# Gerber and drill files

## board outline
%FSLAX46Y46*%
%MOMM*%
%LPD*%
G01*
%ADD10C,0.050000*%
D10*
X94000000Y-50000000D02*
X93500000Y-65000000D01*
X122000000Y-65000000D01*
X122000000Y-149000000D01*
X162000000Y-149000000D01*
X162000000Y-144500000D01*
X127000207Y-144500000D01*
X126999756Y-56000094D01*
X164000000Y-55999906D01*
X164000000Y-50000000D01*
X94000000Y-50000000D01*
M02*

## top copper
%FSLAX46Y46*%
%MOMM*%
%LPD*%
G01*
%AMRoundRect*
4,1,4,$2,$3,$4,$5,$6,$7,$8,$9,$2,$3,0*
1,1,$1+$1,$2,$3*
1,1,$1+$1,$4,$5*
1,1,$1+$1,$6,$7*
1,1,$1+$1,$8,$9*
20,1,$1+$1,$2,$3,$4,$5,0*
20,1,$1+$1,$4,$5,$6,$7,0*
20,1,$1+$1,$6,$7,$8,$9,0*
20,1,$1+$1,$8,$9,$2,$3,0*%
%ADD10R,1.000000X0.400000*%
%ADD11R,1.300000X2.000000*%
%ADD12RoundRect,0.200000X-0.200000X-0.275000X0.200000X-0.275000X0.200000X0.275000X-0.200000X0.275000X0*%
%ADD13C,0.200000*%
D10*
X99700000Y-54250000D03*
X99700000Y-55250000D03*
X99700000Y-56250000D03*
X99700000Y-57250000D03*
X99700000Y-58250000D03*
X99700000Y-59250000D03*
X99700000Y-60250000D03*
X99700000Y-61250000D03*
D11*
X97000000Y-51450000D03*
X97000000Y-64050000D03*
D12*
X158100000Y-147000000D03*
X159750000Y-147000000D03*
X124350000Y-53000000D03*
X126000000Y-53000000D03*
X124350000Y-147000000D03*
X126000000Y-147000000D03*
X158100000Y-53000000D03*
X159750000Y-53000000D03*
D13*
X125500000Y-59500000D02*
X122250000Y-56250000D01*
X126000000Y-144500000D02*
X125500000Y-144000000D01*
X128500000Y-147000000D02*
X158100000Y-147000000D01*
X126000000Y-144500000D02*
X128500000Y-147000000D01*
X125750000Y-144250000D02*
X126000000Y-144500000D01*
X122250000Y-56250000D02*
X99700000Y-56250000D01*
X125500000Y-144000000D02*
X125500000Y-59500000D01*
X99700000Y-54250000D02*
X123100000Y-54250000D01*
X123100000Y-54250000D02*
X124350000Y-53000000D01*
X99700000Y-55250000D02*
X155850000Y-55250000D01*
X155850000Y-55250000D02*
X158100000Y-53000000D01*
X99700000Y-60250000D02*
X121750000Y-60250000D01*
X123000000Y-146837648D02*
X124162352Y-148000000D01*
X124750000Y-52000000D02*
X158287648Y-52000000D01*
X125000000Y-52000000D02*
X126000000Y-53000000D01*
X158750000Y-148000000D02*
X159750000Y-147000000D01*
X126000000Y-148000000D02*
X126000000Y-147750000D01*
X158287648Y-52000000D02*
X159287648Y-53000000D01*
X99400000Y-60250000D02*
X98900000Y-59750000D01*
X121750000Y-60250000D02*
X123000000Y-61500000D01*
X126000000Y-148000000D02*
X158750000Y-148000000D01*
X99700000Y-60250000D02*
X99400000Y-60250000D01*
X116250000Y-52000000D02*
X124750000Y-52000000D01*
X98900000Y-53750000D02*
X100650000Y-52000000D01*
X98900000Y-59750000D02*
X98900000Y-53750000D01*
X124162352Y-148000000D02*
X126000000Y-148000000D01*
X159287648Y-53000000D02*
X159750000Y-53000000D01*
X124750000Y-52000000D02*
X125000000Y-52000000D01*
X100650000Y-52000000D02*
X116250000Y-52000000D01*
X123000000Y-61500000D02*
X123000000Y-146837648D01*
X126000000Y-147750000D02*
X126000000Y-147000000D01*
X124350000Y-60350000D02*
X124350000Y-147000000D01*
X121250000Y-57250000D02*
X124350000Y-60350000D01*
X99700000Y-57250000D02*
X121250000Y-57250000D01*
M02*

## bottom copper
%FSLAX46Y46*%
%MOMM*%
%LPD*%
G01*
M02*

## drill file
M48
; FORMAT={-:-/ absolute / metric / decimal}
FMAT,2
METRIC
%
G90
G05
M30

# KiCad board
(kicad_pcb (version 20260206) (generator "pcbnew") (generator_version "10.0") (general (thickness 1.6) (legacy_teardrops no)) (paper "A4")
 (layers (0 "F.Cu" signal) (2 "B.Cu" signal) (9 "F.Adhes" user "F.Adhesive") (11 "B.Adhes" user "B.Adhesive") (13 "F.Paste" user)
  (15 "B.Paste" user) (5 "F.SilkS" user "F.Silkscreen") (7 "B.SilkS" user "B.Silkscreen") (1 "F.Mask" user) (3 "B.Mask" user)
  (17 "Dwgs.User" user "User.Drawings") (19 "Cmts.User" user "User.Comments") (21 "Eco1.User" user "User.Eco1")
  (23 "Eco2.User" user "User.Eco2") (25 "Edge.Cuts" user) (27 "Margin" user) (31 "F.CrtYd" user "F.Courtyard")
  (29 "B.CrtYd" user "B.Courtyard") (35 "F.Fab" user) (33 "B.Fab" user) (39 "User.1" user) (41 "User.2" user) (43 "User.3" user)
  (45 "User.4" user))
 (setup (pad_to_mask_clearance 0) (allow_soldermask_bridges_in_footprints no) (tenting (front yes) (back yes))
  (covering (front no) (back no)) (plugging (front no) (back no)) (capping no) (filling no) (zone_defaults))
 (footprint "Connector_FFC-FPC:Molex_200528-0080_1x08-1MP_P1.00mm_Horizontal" (layer "F.Cu") (at 98.79 57.75 -90)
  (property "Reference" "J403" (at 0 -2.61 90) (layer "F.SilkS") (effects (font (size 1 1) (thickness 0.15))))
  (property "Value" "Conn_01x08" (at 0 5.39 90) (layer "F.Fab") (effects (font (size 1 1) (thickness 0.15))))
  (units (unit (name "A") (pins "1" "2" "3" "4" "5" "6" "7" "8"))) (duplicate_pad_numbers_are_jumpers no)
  (pad "1" smd rect (at -3.5 -0.91 270) (size 0.4 1) (layers "F.Cu" "F.Mask" "F.Paste") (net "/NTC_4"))
  (pad "2" smd rect (at -2.5 -0.91 270) (size 0.4 1) (layers "F.Cu" "F.Mask" "F.Paste") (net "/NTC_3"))
  (pad "3" smd rect (at -1.5 -0.91 270) (size 0.4 1) (layers "F.Cu" "F.Mask" "F.Paste") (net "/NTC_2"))
  (pad "4" smd rect (at -0.5 -0.91 270) (size 0.4 1) (layers "F.Cu" "F.Mask" "F.Paste") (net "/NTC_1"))
  (pad "5" smd rect (at 0.5 -0.91 270) (size 0.4 1) (layers "F.Cu" "F.Mask" "F.Paste") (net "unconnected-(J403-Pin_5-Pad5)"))
  (pad "6" smd rect (at 1.5 -0.91 270) (size 0.4 1) (layers "F.Cu" "F.Mask" "F.Paste") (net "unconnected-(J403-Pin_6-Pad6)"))
  (pad "7" smd rect (at 2.5 -0.91 270) (size 0.4 1) (layers "F.Cu" "F.Mask" "F.Paste") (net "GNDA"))
  (pad "8" smd rect (at 3.5 -0.91 270) (size 0.4 1) (layers "F.Cu" "F.Mask" "F.Paste") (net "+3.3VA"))
  (pad "MP" smd rect (at -6.3 1.79 270) (size 2 1.3) (layers "F.Cu" "F.Mask" "F.Paste"))
  (pad "MP" smd rect (at 6.3 1.79 270) (size 2 1.3) (layers "F.Cu" "F.Mask" "F.Paste")))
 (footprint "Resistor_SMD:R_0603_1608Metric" (layer "F.Cu") (at 158.925 147)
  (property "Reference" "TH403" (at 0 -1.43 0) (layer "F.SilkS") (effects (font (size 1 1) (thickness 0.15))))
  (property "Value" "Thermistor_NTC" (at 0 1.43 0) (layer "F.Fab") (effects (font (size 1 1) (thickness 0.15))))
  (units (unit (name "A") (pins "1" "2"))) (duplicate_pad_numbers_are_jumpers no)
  (pad "1" smd roundrect (at -0.825 0) (size 0.8 0.95) (layers "F.Cu" "F.Mask" "F.Paste") (roundrect_rratio 0.25) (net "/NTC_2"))
  (pad "2" smd roundrect (at 0.825 0) (size 0.8 0.95) (layers "F.Cu" "F.Mask" "F.Paste") (roundrect_rratio 0.25) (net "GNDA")))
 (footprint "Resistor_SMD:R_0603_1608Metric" (layer "F.Cu") (at 125.175 53)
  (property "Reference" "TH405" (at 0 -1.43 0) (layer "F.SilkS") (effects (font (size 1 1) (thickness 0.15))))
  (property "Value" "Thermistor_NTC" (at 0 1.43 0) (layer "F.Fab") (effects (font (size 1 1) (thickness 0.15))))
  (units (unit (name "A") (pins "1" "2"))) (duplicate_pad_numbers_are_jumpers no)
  (pad "1" smd roundrect (at -0.825 0) (size 0.8 0.95) (layers "F.Cu" "F.Mask" "F.Paste") (roundrect_rratio 0.25) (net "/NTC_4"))
  (pad "2" smd roundrect (at 0.825 0) (size 0.8 0.95) (layers "F.Cu" "F.Mask" "F.Paste") (roundrect_rratio 0.25) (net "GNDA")))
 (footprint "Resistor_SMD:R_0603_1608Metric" (layer "F.Cu") (at 125.175 147)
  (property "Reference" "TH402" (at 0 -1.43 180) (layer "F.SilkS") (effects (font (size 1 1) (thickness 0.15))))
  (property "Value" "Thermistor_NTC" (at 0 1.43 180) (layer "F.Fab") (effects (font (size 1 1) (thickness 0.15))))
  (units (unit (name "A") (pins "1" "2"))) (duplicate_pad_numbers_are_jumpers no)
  (pad "1" smd roundrect (at -0.825 0) (size 0.8 0.95) (layers "F.Cu" "F.Mask" "F.Paste") (roundrect_rratio 0.25) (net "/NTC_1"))
  (pad "2" smd roundrect (at 0.825 0) (size 0.8 0.95) (layers "F.Cu" "F.Mask" "F.Paste") (roundrect_rratio 0.25) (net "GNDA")))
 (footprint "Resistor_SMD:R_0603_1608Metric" (layer "F.Cu") (at 158.925 53)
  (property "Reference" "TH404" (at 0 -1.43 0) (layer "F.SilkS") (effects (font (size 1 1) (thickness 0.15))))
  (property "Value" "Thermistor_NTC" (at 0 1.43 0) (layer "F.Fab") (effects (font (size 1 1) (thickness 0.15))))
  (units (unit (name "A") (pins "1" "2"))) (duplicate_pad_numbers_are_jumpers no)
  (pad "1" smd roundrect (at -0.825 0) (size 0.8 0.95) (layers "F.Cu" "F.Mask" "F.Paste") (roundrect_rratio 0.25) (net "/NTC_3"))
  (pad "2" smd roundrect (at 0.825 0) (size 0.8 0.95) (layers "F.Cu" "F.Mask" "F.Paste") (roundrect_rratio 0.25) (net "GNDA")))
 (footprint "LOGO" (layer "F.Cu") (at 109 57)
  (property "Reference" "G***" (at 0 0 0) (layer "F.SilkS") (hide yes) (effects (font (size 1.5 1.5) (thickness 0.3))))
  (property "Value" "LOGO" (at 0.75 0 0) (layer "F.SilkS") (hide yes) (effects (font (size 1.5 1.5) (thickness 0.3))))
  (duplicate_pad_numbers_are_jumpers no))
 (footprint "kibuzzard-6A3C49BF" (layer "B.Cu") (at 96.5 57.5 90)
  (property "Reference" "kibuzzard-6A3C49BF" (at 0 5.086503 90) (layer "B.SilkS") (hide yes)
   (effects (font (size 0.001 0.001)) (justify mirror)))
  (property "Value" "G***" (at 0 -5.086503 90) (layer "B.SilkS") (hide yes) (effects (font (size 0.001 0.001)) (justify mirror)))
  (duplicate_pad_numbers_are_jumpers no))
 (gr_poly
  (pts (xy 94 50) (xy 93.5 65) (xy 122 65) (xy 122 149) (xy 162 149) (xy 162 144.5) (xy 127.000207 144.5) (xy 126.999756 56.000094)
   (xy 164 55.999906) (xy 164 50))
  (stroke (width 0.05) (type solid)) (fill no) (layer "Edge.Cuts"))
 (segment (start 125.5 59.5) (end 122.25 56.25) (width 0.2) (layer "F.Cu") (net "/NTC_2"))
 (segment (start 126 144.5) (end 125.5 144) (width 0.2) (layer "F.Cu") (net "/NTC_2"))
 (segment (start 128.5 147) (end 158.1 147) (width 0.2) (layer "F.Cu") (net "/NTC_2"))
 (segment (start 126 144.5) (end 128.5 147) (width 0.2) (layer "F.Cu") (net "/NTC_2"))
 (segment (start 125.75 144.25) (end 126 144.5) (width 0.2) (layer "F.Cu") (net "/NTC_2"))
 (segment (start 122.25 56.25) (end 99.7 56.25) (width 0.2) (layer "F.Cu") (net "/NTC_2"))
 (segment (start 125.5 144) (end 125.5 59.5) (width 0.2) (layer "F.Cu") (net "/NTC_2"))
 (segment (start 99.7 54.25) (end 123.1 54.25) (width 0.2) (layer "F.Cu") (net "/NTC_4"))
 (segment (start 123.1 54.25) (end 124.35 53) (width 0.2) (layer "F.Cu") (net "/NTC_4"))
 (segment (start 99.7 55.25) (end 155.85 55.25) (width 0.2) (layer "F.Cu") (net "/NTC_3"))
 (segment (start 155.85 55.25) (end 158.1 53) (width 0.2) (layer "F.Cu") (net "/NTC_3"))
 (segment (start 99.7 60.25) (end 121.75 60.25) (width 0.2) (layer "F.Cu") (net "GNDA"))
 (segment (start 123 146.837648) (end 124.162352 148) (width 0.2) (layer "F.Cu") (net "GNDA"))
 (segment (start 124.75 52) (end 158.287648 52) (width 0.2) (layer "F.Cu") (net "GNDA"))
 (segment (start 125 52) (end 126 53) (width 0.2) (layer "F.Cu") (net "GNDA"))
 (segment (start 158.75 148) (end 159.75 147) (width 0.2) (layer "F.Cu") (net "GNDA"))
 (segment (start 126 148) (end 126 147.75) (width 0.2) (layer "F.Cu") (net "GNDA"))
 (segment (start 158.287648 52) (end 159.287648 53) (width 0.2) (layer "F.Cu") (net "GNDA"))
 (segment (start 99.4 60.25) (end 98.9 59.75) (width 0.2) (layer "F.Cu") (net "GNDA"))
 (segment (start 121.75 60.25) (end 123 61.5) (width 0.2) (layer "F.Cu") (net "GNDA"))
 (segment (start 126 148) (end 158.75 148) (width 0.2) (layer "F.Cu") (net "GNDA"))
 (segment (start 99.7 60.25) (end 99.4 60.25) (width 0.2) (layer "F.Cu") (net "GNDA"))
 (segment (start 116.25 52) (end 124.75 52) (width 0.2) (layer "F.Cu") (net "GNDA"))
 (segment (start 98.9 53.75) (end 100.65 52) (width 0.2) (layer "F.Cu") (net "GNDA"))
 (segment (start 98.9 59.75) (end 98.9 53.75) (width 0.2) (layer "F.Cu") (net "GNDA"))
 (segment (start 124.162352 148) (end 126 148) (width 0.2) (layer "F.Cu") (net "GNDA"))
 (segment (start 159.287648 53) (end 159.75 53) (width 0.2) (layer "F.Cu") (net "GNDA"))
 (segment (start 124.75 52) (end 125 52) (width 0.2) (layer "F.Cu") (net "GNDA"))
 (segment (start 100.65 52) (end 116.25 52) (width 0.2) (layer "F.Cu") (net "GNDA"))
 (segment (start 123 61.5) (end 123 146.837648) (width 0.2) (layer "F.Cu") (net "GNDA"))
 (segment (start 126 147.75) (end 126 147) (width 0.2) (layer "F.Cu") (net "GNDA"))
 (segment (start 124.35 60.35) (end 124.35 147) (width 0.2) (layer "F.Cu") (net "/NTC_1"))
 (segment (start 121.25 57.25) (end 124.35 60.35) (width 0.2) (layer "F.Cu") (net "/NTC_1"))
 (segment (start 99.7 57.25) (end 121.25 57.25) (width 0.2) (layer "F.Cu") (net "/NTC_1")))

